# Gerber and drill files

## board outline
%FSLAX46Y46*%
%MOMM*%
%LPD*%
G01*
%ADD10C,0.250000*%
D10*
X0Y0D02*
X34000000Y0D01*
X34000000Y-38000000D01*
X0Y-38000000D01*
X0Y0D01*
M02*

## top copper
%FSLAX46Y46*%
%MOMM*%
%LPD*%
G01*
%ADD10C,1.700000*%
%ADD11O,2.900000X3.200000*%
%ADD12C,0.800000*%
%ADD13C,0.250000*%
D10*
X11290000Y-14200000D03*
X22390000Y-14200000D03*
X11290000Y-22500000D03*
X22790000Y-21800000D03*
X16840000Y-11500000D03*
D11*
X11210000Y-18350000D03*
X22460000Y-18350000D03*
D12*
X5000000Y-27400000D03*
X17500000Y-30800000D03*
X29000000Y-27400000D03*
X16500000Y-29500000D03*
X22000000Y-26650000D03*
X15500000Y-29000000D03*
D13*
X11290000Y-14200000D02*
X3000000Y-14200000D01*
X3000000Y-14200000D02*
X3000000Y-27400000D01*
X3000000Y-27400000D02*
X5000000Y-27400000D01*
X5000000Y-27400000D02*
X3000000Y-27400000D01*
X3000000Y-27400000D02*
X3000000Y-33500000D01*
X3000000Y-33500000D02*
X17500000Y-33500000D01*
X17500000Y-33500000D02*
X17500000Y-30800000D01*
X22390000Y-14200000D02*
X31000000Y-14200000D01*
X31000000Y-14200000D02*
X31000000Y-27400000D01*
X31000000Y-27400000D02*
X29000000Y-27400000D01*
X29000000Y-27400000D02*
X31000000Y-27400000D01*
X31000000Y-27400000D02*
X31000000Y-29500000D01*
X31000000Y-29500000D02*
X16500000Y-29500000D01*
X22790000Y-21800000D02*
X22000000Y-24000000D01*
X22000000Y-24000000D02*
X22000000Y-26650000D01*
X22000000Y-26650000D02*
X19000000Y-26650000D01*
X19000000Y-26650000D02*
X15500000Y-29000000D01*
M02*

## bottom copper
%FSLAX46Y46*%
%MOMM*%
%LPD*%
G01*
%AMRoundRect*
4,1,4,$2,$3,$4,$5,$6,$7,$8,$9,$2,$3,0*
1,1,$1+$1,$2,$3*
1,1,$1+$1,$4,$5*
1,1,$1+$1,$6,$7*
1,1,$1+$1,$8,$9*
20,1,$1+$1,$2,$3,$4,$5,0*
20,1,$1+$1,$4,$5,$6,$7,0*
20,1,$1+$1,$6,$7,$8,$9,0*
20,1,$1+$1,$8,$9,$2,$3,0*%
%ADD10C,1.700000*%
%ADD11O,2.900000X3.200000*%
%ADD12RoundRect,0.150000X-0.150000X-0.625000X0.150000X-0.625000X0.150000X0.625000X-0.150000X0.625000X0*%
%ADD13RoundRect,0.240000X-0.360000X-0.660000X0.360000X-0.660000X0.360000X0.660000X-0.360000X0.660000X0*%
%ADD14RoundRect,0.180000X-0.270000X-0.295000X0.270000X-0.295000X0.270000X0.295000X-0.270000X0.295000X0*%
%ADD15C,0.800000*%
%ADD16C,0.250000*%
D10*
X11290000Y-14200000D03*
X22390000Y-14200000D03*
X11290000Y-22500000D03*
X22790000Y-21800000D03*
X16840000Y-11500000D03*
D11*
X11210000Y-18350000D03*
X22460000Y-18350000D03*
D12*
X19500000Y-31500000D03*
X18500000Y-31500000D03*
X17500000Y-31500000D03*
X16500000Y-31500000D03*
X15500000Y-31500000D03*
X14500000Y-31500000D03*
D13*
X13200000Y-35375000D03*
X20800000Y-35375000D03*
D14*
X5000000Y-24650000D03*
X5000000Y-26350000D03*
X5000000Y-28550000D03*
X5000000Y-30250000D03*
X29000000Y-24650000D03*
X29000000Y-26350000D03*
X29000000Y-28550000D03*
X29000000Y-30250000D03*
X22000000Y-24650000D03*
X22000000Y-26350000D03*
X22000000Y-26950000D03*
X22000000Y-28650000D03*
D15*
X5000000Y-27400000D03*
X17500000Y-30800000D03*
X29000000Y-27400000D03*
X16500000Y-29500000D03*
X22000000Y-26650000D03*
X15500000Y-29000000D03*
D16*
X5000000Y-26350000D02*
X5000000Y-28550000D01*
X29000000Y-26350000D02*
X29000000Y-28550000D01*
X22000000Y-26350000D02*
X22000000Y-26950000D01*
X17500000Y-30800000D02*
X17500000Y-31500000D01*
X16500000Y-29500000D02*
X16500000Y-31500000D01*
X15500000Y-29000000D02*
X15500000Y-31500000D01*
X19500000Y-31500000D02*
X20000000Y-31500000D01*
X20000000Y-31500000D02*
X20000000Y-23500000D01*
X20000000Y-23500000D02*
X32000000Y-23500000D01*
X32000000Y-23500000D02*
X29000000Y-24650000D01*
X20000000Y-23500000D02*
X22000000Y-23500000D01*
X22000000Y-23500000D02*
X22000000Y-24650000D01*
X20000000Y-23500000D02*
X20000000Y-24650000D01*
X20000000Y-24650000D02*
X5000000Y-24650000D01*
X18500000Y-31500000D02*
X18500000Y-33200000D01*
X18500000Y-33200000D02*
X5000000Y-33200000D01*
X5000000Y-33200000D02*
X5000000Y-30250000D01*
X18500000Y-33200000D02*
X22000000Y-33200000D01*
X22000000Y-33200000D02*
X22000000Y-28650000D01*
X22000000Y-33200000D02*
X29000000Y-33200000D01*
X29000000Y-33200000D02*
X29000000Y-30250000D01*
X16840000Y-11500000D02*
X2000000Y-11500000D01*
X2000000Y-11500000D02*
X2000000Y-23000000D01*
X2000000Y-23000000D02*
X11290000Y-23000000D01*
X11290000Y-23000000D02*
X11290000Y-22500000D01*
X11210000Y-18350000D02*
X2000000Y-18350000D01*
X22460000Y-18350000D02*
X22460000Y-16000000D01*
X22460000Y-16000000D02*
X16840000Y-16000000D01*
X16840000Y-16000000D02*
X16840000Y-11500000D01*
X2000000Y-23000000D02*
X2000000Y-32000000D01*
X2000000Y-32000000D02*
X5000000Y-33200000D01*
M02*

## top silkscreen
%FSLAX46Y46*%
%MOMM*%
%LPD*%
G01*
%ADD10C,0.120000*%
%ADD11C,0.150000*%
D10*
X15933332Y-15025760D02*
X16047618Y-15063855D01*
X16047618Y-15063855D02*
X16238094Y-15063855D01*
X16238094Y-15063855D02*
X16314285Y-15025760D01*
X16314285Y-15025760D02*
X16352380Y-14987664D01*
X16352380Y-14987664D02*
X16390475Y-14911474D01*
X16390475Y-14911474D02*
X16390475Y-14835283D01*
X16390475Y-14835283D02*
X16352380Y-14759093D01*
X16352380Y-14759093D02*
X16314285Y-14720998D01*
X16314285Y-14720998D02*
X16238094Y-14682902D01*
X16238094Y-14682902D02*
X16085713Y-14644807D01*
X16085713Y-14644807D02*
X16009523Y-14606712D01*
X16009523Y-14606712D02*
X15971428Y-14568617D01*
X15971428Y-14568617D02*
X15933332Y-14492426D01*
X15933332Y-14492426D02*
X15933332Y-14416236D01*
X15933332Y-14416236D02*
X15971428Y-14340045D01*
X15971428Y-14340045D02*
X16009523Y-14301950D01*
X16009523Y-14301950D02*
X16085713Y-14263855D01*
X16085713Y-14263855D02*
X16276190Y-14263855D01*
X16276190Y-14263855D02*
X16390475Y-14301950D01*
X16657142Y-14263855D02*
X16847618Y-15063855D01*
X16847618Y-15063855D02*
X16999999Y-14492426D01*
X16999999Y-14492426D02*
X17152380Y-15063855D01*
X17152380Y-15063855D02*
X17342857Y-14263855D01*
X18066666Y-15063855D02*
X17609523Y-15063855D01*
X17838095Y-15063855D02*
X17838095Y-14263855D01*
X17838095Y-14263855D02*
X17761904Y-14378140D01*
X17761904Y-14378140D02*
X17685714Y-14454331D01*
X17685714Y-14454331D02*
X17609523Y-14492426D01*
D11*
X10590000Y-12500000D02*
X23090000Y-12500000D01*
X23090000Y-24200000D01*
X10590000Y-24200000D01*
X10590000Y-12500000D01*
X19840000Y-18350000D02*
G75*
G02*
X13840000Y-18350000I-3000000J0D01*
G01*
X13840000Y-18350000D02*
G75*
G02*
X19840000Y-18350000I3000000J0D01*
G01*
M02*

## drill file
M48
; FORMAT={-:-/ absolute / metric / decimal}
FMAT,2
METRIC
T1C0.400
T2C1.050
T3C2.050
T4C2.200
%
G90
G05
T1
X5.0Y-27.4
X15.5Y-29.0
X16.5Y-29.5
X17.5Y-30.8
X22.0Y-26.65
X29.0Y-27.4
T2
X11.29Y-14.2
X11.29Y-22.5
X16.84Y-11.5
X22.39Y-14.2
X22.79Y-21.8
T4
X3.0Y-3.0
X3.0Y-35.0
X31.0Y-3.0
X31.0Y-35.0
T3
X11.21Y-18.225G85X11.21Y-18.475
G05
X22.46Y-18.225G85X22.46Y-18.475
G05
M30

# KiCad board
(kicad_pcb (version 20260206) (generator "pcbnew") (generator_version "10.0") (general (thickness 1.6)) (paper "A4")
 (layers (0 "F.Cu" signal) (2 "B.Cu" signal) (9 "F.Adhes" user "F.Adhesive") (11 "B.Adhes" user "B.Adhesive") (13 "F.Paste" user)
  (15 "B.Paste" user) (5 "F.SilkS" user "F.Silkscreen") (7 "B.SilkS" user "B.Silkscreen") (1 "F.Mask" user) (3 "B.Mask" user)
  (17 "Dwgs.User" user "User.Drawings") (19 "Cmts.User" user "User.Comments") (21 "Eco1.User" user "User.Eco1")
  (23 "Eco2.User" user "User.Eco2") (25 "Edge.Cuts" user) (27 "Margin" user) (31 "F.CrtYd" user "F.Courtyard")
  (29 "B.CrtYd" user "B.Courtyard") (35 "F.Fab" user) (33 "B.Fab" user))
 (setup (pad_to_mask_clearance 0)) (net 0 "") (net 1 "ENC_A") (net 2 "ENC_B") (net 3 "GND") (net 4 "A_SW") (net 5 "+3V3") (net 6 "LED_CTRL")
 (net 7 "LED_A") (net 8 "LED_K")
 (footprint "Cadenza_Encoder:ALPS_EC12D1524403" (layer "F.Cu") (at 17.000 17.000)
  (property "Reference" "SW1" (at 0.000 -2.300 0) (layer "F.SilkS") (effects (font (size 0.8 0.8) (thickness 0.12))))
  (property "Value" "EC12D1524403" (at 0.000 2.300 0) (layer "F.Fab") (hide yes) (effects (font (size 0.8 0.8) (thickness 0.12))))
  (fp_rect (start -6.41 -4.50) (end 6.09 7.20) (stroke (width 0.15) (type solid)) (fill none) (layer "F.SilkS"))
  (fp_circle (center -0.16 1.35) (end 2.84 1.35) (stroke (width 0.15) (type solid)) (fill none) (layer "F.SilkS"))
  (pad "A" thru_hole circle (at -5.710 -2.800) (size 1.700 1.700) (drill 1.05) (layers "*.Cu" "*.Mask") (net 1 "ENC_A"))
  (pad "B" thru_hole circle (at 5.390 -2.800) (size 1.700 1.700) (drill 1.05) (layers "*.Cu" "*.Mask") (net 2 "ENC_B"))
  (pad "C" thru_hole circle (at -5.710 5.500) (size 1.700 1.700) (drill 1.05) (layers "*.Cu" "*.Mask") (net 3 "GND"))
  (pad "D" thru_hole circle (at 5.790 4.800) (size 1.700 1.700) (drill 1.05) (layers "*.Cu" "*.Mask") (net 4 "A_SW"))
  (pad "E" thru_hole circle (at -0.160 -5.500) (size 1.700 1.700) (drill 1.05) (layers "*.Cu" "*.Mask") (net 3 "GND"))
  (pad "6" thru_hole oval (at -5.790 1.350) (size 2.900 3.200) (drill oval 2.05 2.30) (layers "*.Cu" "*.Mask") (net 3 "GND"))
  (pad "7" thru_hole oval (at 5.460 1.350) (size 2.900 3.200) (drill oval 2.05 2.30) (layers "*.Cu" "*.Mask") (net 3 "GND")))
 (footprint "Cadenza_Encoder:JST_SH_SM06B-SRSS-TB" (layer "B.Cu") (at 17.000 33.500)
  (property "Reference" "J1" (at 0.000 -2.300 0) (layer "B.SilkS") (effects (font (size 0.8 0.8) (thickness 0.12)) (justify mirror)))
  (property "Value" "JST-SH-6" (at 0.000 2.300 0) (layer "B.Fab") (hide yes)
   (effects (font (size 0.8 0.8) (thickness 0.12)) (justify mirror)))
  (pad "1" smd roundrect (at 2.500 -2.000) (size 0.600 1.550) (layers "B.Cu" "B.Paste" "B.Mask") (roundrect_rratio 0.25) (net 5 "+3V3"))
  (pad "2" smd roundrect (at 1.500 -2.000) (size 0.600 1.550) (layers "B.Cu" "B.Paste" "B.Mask") (roundrect_rratio 0.25) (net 3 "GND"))
  (pad "3" smd roundrect (at 0.500 -2.000) (size 0.600 1.550) (layers "B.Cu" "B.Paste" "B.Mask") (roundrect_rratio 0.25) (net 1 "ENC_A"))
  (pad "4" smd roundrect (at -0.500 -2.000) (size 0.600 1.550) (layers "B.Cu" "B.Paste" "B.Mask") (roundrect_rratio 0.25) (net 2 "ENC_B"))
  (pad "5" smd roundrect (at -1.500 -2.000) (size 0.600 1.550) (layers "B.Cu" "B.Paste" "B.Mask") (roundrect_rratio 0.25) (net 4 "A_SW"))
  (pad "6" smd roundrect (at -2.500 -2.000) (size 0.600 1.550) (layers "B.Cu" "B.Paste" "B.Mask") (roundrect_rratio 0.25) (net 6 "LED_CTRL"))
  (pad "MP" smd roundrect (at -3.800 1.875) (size 1.200 1.800) (layers "B.Cu" "B.Paste" "B.Mask") (roundrect_rratio 0.2))
  (pad "MP" smd roundrect (at 3.800 1.875) (size 1.200 1.800) (layers "B.Cu" "B.Paste" "B.Mask") (roundrect_rratio 0.2)))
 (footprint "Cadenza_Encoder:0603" (layer "B.Cu") (at 5.000 25.500)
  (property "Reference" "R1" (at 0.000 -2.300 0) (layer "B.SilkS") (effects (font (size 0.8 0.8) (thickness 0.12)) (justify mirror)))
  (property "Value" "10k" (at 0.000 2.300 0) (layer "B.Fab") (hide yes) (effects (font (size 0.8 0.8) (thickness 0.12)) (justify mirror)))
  (pad "1" smd roundrect (at 0.000 -0.850) (size 0.900 0.950) (layers "B.Cu" "B.Paste" "B.Mask") (roundrect_rratio 0.2) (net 5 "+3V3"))
  (pad "2" smd roundrect (at 0.000 0.850) (size 0.900 0.950) (layers "B.Cu" "B.Paste" "B.Mask") (roundrect_rratio 0.2) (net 1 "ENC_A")))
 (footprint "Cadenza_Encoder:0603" (layer "B.Cu") (at 5.000 29.400)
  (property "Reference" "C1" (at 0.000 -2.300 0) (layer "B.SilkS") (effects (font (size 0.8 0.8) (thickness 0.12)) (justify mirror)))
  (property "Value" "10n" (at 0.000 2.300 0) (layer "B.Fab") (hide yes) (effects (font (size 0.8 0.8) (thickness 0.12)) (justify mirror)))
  (pad "1" smd roundrect (at 0.000 -0.850) (size 0.900 0.950) (layers "B.Cu" "B.Paste" "B.Mask") (roundrect_rratio 0.2) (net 1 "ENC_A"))
  (pad "2" smd roundrect (at 0.000 0.850) (size 0.900 0.950) (layers "B.Cu" "B.Paste" "B.Mask") (roundrect_rratio 0.2) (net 3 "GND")))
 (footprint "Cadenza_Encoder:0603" (layer "B.Cu") (at 29.000 25.500)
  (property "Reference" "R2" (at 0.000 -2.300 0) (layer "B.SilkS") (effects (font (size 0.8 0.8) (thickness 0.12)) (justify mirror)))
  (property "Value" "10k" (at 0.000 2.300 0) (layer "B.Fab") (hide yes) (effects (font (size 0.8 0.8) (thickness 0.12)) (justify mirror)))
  (pad "1" smd roundrect (at 0.000 -0.850) (size 0.900 0.950) (layers "B.Cu" "B.Paste" "B.Mask") (roundrect_rratio 0.2) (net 5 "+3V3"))
  (pad "2" smd roundrect (at 0.000 0.850) (size 0.900 0.950) (layers "B.Cu" "B.Paste" "B.Mask") (roundrect_rratio 0.2) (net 2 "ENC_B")))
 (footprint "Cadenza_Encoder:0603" (layer "B.Cu") (at 29.000 29.400)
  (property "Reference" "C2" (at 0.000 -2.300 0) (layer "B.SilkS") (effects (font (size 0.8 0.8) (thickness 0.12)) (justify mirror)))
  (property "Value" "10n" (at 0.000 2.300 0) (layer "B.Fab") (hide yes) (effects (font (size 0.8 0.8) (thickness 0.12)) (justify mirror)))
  (pad "1" smd roundrect (at 0.000 -0.850) (size 0.900 0.950) (layers "B.Cu" "B.Paste" "B.Mask") (roundrect_rratio 0.2) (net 2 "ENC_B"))
  (pad "2" smd roundrect (at 0.000 0.850) (size 0.900 0.950) (layers "B.Cu" "B.Paste" "B.Mask") (roundrect_rratio 0.2) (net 3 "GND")))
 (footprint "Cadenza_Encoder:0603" (layer "B.Cu") (at 22.000 25.500)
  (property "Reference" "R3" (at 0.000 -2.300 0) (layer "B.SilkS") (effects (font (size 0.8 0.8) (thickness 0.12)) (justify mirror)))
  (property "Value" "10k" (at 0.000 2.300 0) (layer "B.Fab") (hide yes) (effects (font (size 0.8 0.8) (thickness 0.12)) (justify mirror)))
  (pad "1" smd roundrect (at 0.000 -0.850) (size 0.900 0.950) (layers "B.Cu" "B.Paste" "B.Mask") (roundrect_rratio 0.2) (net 5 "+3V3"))
  (pad "2" smd roundrect (at 0.000 0.850) (size 0.900 0.950) (layers "B.Cu" "B.Paste" "B.Mask") (roundrect_rratio 0.2) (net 4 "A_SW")))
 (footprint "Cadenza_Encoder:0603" (layer "B.Cu") (at 22.000 27.800)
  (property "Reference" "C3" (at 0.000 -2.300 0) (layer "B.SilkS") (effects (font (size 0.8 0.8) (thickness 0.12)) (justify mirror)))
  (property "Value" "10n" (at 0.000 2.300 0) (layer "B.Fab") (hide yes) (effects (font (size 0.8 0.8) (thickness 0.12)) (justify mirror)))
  (pad "1" smd roundrect (at 0.000 -0.850) (size 0.900 0.950) (layers "B.Cu" "B.Paste" "B.Mask") (roundrect_rratio 0.2) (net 4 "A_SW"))
  (pad "2" smd roundrect (at 0.000 0.850) (size 0.900 0.950) (layers "B.Cu" "B.Paste" "B.Mask") (roundrect_rratio 0.2) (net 3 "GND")))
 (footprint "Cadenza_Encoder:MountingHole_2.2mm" (layer "F.Cu") (at 3 3)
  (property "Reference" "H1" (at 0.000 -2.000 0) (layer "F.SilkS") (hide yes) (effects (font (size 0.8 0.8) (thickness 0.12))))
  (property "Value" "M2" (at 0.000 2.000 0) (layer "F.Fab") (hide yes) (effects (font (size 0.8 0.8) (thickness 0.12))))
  (pad "" np_thru_hole circle (at 0.000 0.000) (size 2.200 2.200) (drill 2.2) (layers "*.Cu" "*.Mask")))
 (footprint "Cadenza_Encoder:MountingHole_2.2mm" (layer "F.Cu") (at 31 3)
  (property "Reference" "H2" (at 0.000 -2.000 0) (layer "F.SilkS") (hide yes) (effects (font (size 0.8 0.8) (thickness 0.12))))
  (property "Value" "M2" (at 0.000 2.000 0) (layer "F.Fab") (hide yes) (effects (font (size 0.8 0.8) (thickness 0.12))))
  (pad "" np_thru_hole circle (at 0.000 0.000) (size 2.200 2.200) (drill 2.2) (layers "*.Cu" "*.Mask")))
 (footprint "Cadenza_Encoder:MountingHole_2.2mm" (layer "F.Cu") (at 3 35)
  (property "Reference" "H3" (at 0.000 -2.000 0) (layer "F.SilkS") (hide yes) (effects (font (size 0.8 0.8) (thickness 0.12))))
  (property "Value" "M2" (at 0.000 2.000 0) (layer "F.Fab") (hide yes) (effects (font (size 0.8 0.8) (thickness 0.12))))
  (pad "" np_thru_hole circle (at 0.000 0.000) (size 2.200 2.200) (drill 2.2) (layers "*.Cu" "*.Mask")))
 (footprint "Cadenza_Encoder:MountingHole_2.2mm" (layer "F.Cu") (at 31 35)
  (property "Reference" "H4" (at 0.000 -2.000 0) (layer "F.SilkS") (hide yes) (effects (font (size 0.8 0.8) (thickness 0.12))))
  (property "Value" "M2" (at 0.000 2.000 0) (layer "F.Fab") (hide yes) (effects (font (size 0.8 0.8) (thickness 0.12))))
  (pad "" np_thru_hole circle (at 0.000 0.000) (size 2.200 2.200) (drill 2.2) (layers "*.Cu" "*.Mask")))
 (segment (start 5.000 26.350) (end 5.000 28.550) (width 0.25) (layer "B.Cu") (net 1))
 (segment (start 29.000 26.350) (end 29.000 28.550) (width 0.25) (layer "B.Cu") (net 2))
 (segment (start 22.000 26.350) (end 22.000 26.950) (width 0.25) (layer "B.Cu") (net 4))
 (segment (start 11.290 14.200) (end 3.000 14.200) (width 0.25) (layer "F.Cu") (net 1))
 (segment (start 3.000 14.200) (end 3.000 27.400) (width 0.25) (layer "F.Cu") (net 1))
 (segment (start 3.000 27.400) (end 5.000 27.400) (width 0.25) (layer "F.Cu") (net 1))
 (segment (start 5.000 27.400) (end 3.000 27.400) (width 0.25) (layer "F.Cu") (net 1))
 (segment (start 3.000 27.400) (end 3.000 33.500) (width 0.25) (layer "F.Cu") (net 1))
 (segment (start 3.000 33.500) (end 17.500 33.500) (width 0.25) (layer "F.Cu") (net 1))
 (segment (start 17.500 33.500) (end 17.500 30.800) (width 0.25) (layer "F.Cu") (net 1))
 (segment (start 17.500 30.800) (end 17.500 31.500) (width 0.25) (layer "B.Cu") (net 1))
 (segment (start 22.390 14.200) (end 31.000 14.200) (width 0.25) (layer "F.Cu") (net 2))
 (segment (start 31.000 14.200) (end 31.000 27.400) (width 0.25) (layer "F.Cu") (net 2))
 (segment (start 31.000 27.400) (end 29.000 27.400) (width 0.25) (layer "F.Cu") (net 2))
 (segment (start 29.000 27.400) (end 31.000 27.400) (width 0.25) (layer "F.Cu") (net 2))
 (segment (start 31.000 27.400) (end 31.000 29.500) (width 0.25) (layer "F.Cu") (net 2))
 (segment (start 31.000 29.500) (end 16.500 29.500) (width 0.25) (layer "F.Cu") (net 2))
 (segment (start 16.500 29.500) (end 16.500 31.500) (width 0.25) (layer "B.Cu") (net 2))
 (segment (start 22.790 21.800) (end 22.000 24.000) (width 0.25) (layer "F.Cu") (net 4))
 (segment (start 22.000 24.000) (end 22.000 26.650) (width 0.25) (layer "F.Cu") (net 4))
 (segment (start 22.000 26.650) (end 19.000 26.650) (width 0.25) (layer "F.Cu") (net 4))
 (segment (start 19.000 26.650) (end 15.500 29.000) (width 0.25) (layer "F.Cu") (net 4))
 (segment (start 15.500 29.000) (end 15.500 31.500) (width 0.25) (layer "B.Cu") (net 4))
 (segment (start 19.500 31.500) (end 20.000 31.500) (width 0.25) (layer "B.Cu") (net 5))
 (segment (start 20.000 31.500) (end 20.000 23.500) (width 0.25) (layer "B.Cu") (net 5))
 (segment (start 20.000 23.500) (end 32.000 23.500) (width 0.25) (layer "B.Cu") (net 5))
 (segment (start 32.000 23.500) (end 29.000 24.650) (width 0.25) (layer "B.Cu") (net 5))
 (segment (start 20.000 23.500) (end 22.000 23.500) (width 0.25) (layer "B.Cu") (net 5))
 (segment (start 22.000 23.500) (end 22.000 24.650) (width 0.25) (layer "B.Cu") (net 5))
 (segment (start 20.000 23.500) (end 20.000 24.650) (width 0.25) (layer "B.Cu") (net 5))
 (segment (start 20.000 24.650) (end 5.000 24.650) (width 0.25) (layer "B.Cu") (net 5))
 (segment (start 18.500 31.500) (end 18.500 33.200) (width 0.25) (layer "B.Cu") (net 3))
 (segment (start 18.500 33.200) (end 5.000 33.200) (width 0.25) (layer "B.Cu") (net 3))
 (segment (start 5.000 33.200) (end 5.000 30.250) (width 0.25) (layer "B.Cu") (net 3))
 (segment (start 18.500 33.200) (end 22.000 33.200) (width 0.25) (layer "B.Cu") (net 3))
 (segment (start 22.000 33.200) (end 22.000 28.650) (width 0.25) (layer "B.Cu") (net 3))
 (segment (start 22.000 33.200) (end 29.000 33.200) (width 0.25) (layer "B.Cu") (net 3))
 (segment (start 29.000 33.200) (end 29.000 30.250) (width 0.25) (layer "B.Cu") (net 3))
 (segment (start 16.840 11.500) (end 2.000 11.500) (width 0.25) (layer "B.Cu") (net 3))
 (segment (start 2.000 11.500) (end 2.000 23.000) (width 0.25) (layer "B.Cu") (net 3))
 (segment (start 2.000 23.000) (end 11.290 23.000) (width 0.25) (layer "B.Cu") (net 3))
 (segment (start 11.290 23.000) (end 11.290 22.500) (width 0.25) (layer "B.Cu") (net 3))
 (segment (start 11.210 18.350) (end 2.000 18.350) (width 0.25) (layer "B.Cu") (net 3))
 (segment (start 22.460 18.350) (end 22.460 16.000) (width 0.25) (layer "B.Cu") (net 3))
 (segment (start 22.460 16.000) (end 16.840 16.000) (width 0.25) (layer "B.Cu") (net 3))
 (segment (start 16.840 16.000) (end 16.840 11.500) (width 0.25) (layer "B.Cu") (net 3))
 (segment (start 2.000 23.000) (end 2.000 32.000) (width 0.25) (layer "B.Cu") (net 3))
 (segment (start 2.000 32.000) (end 5.000 33.200) (width 0.25) (layer "B.Cu") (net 3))
 (via (at 5.000 27.400) (size 0.8) (drill 0.4) (layers "F.Cu" "B.Cu") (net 1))
 (via (at 17.500 30.800) (size 0.8) (drill 0.4) (layers "F.Cu" "B.Cu") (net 1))
 (via (at 29.000 27.400) (size 0.8) (drill 0.4) (layers "F.Cu" "B.Cu") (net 2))
 (via (at 16.500 29.500) (size 0.8) (drill 0.4) (layers "F.Cu" "B.Cu") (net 2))
 (via (at 22.000 26.650) (size 0.8) (drill 0.4) (layers "F.Cu" "B.Cu") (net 4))
 (via (at 15.500 29.000) (size 0.8) (drill 0.4) (layers "F.Cu" "B.Cu") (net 4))
 (gr_rect (start 0 0) (end 34 38) (stroke (width 0.25) (type solid)) (fill none) (layer "Edge.Cuts")))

